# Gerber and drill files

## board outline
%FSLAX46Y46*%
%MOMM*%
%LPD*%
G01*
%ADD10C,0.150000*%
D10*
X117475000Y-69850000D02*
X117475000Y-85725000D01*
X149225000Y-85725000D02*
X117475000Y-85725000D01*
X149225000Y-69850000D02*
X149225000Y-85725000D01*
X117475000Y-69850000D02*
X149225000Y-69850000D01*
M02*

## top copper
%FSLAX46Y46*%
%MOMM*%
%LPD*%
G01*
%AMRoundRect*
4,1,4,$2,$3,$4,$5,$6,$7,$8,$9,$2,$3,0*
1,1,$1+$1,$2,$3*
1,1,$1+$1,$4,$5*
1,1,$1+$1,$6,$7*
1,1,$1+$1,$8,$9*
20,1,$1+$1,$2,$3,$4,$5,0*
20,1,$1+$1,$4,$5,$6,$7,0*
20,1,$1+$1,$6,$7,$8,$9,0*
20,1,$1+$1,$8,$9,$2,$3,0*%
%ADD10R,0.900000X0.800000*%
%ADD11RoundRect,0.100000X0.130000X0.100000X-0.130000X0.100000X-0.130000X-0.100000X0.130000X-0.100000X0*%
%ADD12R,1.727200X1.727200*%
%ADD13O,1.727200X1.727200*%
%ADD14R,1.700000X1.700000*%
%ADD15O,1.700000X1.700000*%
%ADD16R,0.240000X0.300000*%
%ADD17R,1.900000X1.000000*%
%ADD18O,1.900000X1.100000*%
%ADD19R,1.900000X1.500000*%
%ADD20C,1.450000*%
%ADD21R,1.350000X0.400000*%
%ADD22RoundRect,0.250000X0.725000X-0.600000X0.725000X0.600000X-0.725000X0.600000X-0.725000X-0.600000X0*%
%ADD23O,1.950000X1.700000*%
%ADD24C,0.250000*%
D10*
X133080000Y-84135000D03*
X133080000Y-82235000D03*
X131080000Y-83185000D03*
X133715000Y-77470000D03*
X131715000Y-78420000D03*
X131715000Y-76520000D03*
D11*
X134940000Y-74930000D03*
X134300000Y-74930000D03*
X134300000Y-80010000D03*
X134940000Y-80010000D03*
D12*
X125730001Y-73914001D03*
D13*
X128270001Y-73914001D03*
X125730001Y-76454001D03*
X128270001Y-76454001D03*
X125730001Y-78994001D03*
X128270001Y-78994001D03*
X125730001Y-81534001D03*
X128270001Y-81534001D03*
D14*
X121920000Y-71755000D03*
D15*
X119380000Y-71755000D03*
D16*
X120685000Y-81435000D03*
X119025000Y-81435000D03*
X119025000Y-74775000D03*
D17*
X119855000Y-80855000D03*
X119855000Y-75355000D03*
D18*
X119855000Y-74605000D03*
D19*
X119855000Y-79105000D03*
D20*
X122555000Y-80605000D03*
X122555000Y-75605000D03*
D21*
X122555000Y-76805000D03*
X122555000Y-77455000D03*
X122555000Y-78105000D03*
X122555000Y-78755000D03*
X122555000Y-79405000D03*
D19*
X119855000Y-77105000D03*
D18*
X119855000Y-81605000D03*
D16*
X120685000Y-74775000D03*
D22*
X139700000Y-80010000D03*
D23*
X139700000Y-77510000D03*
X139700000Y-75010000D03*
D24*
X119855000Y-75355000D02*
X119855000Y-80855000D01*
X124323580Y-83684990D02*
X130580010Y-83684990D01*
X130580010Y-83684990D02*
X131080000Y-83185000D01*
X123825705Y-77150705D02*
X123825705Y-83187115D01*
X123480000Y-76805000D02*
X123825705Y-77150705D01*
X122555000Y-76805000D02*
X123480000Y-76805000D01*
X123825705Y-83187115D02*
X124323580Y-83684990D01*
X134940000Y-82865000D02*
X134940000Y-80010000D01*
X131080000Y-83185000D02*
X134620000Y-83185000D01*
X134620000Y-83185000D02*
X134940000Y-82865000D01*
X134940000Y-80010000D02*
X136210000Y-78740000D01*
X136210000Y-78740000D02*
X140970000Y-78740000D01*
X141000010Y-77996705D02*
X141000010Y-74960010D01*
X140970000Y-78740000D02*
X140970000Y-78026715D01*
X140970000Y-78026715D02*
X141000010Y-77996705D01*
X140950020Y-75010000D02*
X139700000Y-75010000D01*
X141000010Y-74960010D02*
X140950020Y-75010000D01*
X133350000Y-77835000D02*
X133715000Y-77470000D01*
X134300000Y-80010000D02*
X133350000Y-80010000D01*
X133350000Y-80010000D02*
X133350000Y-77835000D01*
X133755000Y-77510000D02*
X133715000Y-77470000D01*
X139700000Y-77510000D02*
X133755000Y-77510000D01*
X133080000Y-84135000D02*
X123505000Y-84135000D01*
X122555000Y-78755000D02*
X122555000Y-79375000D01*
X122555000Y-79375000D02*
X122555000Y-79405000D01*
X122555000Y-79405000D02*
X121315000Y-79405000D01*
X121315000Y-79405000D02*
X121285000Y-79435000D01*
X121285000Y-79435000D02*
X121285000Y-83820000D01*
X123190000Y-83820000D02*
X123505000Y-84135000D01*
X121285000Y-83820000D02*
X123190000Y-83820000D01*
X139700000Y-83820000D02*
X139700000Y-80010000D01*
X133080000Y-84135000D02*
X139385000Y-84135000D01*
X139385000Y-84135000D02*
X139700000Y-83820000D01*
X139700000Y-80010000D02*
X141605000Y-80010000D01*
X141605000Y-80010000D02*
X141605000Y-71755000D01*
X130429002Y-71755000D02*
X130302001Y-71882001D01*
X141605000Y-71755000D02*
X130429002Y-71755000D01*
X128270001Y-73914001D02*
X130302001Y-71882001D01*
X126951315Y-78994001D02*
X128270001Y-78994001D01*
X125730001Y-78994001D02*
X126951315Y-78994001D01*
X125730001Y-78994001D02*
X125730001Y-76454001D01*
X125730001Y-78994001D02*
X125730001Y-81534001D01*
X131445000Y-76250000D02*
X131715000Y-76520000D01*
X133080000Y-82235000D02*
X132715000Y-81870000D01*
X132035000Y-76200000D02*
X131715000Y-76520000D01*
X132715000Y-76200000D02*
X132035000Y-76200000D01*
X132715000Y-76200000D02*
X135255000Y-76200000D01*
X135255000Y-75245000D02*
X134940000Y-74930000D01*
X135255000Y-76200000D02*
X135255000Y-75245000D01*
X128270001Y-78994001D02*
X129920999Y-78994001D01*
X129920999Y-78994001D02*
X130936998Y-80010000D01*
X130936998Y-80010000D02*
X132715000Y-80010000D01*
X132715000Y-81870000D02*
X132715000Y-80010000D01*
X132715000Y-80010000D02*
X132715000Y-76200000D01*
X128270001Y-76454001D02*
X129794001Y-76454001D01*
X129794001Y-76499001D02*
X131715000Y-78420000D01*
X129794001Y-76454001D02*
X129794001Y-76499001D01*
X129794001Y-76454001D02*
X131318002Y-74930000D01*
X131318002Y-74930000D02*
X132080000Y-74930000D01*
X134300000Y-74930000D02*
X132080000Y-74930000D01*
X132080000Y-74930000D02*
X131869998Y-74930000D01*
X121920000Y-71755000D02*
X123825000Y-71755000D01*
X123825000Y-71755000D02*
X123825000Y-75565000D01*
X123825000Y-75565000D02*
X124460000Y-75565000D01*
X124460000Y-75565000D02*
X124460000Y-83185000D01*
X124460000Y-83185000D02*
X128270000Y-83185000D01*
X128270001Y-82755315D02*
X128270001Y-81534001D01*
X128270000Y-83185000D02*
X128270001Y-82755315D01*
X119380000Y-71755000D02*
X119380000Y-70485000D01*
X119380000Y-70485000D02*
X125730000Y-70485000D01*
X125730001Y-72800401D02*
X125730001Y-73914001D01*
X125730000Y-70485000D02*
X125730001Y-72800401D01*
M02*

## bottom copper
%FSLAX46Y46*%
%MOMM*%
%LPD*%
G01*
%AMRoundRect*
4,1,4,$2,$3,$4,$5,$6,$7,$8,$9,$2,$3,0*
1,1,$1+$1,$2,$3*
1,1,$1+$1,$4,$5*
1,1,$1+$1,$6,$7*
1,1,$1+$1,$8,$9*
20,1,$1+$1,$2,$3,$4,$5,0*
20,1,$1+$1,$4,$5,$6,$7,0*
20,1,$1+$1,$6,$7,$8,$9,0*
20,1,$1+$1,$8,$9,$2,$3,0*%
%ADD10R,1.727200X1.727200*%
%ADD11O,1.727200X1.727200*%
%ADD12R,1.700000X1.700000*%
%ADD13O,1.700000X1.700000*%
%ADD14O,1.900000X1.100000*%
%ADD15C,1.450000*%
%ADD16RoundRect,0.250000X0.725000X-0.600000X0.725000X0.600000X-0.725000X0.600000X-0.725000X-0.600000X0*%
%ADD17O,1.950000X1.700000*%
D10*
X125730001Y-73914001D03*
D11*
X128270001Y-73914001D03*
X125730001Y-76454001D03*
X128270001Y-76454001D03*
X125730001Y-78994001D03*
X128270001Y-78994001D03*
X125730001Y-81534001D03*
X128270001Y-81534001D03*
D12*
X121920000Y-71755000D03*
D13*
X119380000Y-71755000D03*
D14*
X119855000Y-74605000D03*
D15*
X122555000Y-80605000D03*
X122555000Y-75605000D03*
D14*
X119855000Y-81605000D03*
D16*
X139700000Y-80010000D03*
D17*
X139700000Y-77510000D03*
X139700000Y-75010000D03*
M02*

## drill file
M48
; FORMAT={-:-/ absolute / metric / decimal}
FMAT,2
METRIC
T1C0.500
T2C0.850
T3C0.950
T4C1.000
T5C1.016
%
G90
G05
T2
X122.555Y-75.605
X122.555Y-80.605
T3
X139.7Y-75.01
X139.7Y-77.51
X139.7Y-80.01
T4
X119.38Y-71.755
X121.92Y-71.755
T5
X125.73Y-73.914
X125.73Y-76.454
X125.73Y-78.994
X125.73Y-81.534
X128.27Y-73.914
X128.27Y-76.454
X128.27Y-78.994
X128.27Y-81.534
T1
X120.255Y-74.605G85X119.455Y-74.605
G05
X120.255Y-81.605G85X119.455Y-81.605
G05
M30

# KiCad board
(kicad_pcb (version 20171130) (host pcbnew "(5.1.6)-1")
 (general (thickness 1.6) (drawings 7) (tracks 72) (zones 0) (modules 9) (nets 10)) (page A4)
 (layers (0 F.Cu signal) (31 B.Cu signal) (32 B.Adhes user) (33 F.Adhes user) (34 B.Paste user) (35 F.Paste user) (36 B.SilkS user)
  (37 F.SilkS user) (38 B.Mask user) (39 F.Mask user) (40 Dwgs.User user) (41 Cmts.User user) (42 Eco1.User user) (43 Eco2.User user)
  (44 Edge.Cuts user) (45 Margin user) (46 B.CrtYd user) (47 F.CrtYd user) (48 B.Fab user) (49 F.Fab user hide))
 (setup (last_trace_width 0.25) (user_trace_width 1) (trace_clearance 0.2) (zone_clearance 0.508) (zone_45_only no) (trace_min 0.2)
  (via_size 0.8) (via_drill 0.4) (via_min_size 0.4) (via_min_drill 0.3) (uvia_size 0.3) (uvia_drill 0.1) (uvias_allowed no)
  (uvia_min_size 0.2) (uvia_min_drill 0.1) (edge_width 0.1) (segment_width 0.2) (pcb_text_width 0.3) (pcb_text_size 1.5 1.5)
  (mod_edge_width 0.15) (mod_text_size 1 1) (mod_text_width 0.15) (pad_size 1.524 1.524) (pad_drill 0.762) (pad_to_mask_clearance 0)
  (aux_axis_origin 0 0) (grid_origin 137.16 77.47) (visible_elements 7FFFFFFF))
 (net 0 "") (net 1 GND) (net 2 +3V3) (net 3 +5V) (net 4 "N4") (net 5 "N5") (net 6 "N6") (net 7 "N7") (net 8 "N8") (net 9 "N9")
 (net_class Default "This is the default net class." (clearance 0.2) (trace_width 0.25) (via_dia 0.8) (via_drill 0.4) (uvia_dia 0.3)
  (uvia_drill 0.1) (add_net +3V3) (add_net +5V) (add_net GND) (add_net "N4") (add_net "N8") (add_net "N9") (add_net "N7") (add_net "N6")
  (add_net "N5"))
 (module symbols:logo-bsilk (layer F.Cu) (at 133.35 77.47)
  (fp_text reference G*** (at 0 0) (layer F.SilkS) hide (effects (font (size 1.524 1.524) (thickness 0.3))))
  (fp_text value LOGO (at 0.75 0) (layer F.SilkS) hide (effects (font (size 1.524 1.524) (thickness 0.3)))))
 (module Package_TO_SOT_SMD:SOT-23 (layer F.Cu) (at 132.08 83.185 180)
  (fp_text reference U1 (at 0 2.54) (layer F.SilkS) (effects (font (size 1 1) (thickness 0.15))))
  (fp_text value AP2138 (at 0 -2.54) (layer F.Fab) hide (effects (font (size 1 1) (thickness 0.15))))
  (pad 1 smd rect (at -1 -0.95 180) (size 0.9 0.8) (layers F.Cu F.Paste F.Mask) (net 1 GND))
  (pad 2 smd rect (at -1 0.95 180) (size 0.9 0.8) (layers F.Cu F.Paste F.Mask) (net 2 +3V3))
  (pad 3 smd rect (at 1 0 180) (size 0.9 0.8) (layers F.Cu F.Paste F.Mask) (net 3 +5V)))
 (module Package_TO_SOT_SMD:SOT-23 (layer F.Cu) (at 132.715 77.47)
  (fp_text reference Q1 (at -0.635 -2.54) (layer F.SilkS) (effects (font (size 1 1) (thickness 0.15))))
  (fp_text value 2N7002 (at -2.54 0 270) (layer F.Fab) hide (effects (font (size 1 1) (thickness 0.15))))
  (pad 3 smd rect (at 1 0) (size 0.9 0.8) (layers F.Cu F.Paste F.Mask) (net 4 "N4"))
  (pad 2 smd rect (at -1 0.95) (size 0.9 0.8) (layers F.Cu F.Paste F.Mask) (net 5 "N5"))
  (pad 1 smd rect (at -1 -0.95) (size 0.9 0.8) (layers F.Cu F.Paste F.Mask) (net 2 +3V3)))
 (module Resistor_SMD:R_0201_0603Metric (layer F.Cu) (at 134.62 74.93 180)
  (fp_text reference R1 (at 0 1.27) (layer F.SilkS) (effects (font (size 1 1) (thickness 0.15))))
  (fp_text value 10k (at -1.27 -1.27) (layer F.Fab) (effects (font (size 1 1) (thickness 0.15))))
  (pad "" smd roundrect (at -0.345 0 180) (size 0.318 0.36) (layers F.Paste) (roundrect_rratio 0.25))
  (pad "" smd roundrect (at 0.345 0 180) (size 0.318 0.36) (layers F.Paste) (roundrect_rratio 0.25))
  (pad 1 smd roundrect (at -0.32 0 180) (size 0.46 0.4) (layers F.Cu F.Mask) (roundrect_rratio 0.25) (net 2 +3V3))
  (pad 2 smd roundrect (at 0.32 0 180) (size 0.46 0.4) (layers F.Cu F.Mask) (roundrect_rratio 0.25) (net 5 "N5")))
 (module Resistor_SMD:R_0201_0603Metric (layer F.Cu) (at 134.62 80.01 180)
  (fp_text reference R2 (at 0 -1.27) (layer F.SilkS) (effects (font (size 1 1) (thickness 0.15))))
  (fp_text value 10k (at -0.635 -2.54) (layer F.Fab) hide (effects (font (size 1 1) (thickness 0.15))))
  (pad 2 smd roundrect (at 0.32 0 180) (size 0.46 0.4) (layers F.Cu F.Mask) (roundrect_rratio 0.25) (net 4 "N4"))
  (pad 1 smd roundrect (at -0.32 0 180) (size 0.46 0.4) (layers F.Cu F.Mask) (roundrect_rratio 0.25) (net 3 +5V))
  (pad "" smd roundrect (at 0.345 0 180) (size 0.318 0.36) (layers F.Paste) (roundrect_rratio 0.25))
  (pad "" smd roundrect (at -0.345 0 180) (size 0.318 0.36) (layers F.Paste) (roundrect_rratio 0.25)))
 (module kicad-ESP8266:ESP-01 (layer F.Cu) (at 125.730001 73.914001)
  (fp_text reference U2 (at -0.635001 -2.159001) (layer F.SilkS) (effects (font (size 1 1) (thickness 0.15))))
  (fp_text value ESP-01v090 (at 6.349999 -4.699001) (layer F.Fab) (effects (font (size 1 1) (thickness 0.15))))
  (pad 1 thru_hole rect (at 0 0) (size 1.7272 1.7272) (drill 1.016) (layers *.Cu *.Mask F.SilkS) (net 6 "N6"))
  (pad 2 thru_hole oval (at 2.54 0) (size 1.7272 1.7272) (drill 1.016) (layers *.Cu *.Mask F.SilkS) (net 1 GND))
  (pad 3 thru_hole oval (at 0 2.54) (size 1.7272 1.7272) (drill 1.016) (layers *.Cu *.Mask F.SilkS) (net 2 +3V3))
  (pad 4 thru_hole oval (at 2.54 2.54) (size 1.7272 1.7272) (drill 1.016) (layers *.Cu *.Mask F.SilkS) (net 5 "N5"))
  (pad 5 thru_hole oval (at 0 5.08) (size 1.7272 1.7272) (drill 1.016) (layers *.Cu *.Mask F.SilkS) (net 2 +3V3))
  (pad 6 thru_hole oval (at 2.54 5.08) (size 1.7272 1.7272) (drill 1.016) (layers *.Cu *.Mask F.SilkS) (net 2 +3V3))
  (pad 7 thru_hole oval (at 0 7.62) (size 1.7272 1.7272) (drill 1.016) (layers *.Cu *.Mask F.SilkS) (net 2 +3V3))
  (pad 8 thru_hole oval (at 2.54 7.62) (size 1.7272 1.7272) (drill 1.016) (layers *.Cu *.Mask F.SilkS) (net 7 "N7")))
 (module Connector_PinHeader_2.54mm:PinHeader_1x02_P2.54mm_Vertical (layer F.Cu) (at 121.92 71.755 270)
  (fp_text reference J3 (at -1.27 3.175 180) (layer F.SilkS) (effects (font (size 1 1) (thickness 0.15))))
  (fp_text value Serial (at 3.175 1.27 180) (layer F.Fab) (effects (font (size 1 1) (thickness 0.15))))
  (pad 1 thru_hole rect (at 0 0 270) (size 1.7 1.7) (drill 1) (layers *.Cu *.Mask) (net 7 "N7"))
  (pad 2 thru_hole oval (at 0 2.54 270) (size 1.7 1.7) (drill 1) (layers *.Cu *.Mask) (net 6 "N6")))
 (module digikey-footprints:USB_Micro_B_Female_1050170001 (layer F.Cu) (at 122.555 78.105 270)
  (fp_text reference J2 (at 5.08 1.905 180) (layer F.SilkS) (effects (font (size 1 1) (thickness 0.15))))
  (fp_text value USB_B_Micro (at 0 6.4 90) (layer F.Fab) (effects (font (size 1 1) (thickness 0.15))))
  (pad SH smd rect (at 3.33 1.87 270) (size 0.3 0.24) (layers F.Cu F.Paste F.Mask))
  (pad SH smd rect (at 3.33 3.53 270) (size 0.3 0.24) (layers F.Cu F.Paste F.Mask))
  (pad SH smd rect (at -3.33 3.53 270) (size 0.3 0.24) (layers F.Cu F.Paste F.Mask))
  (pad SH smd rect (at 2.75 2.7 270) (size 1 1.9) (layers F.Cu F.Paste F.Mask))
  (pad SH smd rect (at -2.75 2.7 270) (size 1 1.9) (layers F.Cu F.Paste F.Mask))
  (pad SH thru_hole oval (at -3.5 2.7 270) (size 1.1 1.9) (drill oval 0.5 1.3) (layers *.Cu *.Mask))
  (pad SH smd rect (at 1 2.7 270) (size 1.5 1.9) (layers F.Cu F.Paste F.Mask))
  (pad SH thru_hole circle (at 2.5 0 270) (size 1.45 1.45) (drill 0.85) (layers *.Cu *.Mask))
  (pad SH thru_hole circle (at -2.5 0 270) (size 1.45 1.45) (drill 0.85) (layers *.Cu *.Mask))
  (pad 1 smd rect (at -1.3 0 270) (size 0.4 1.35) (layers F.Cu F.Paste F.Mask) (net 3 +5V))
  (pad 2 smd rect (at -0.65 0 270) (size 0.4 1.35) (layers F.Cu F.Paste F.Mask) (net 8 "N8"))
  (pad 3 smd rect (at 0 0 270) (size 0.4 1.35) (layers F.Cu F.Paste F.Mask) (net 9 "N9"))
  (pad 4 smd rect (at 0.65 0 270) (size 0.4 1.35) (layers F.Cu F.Paste F.Mask) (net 1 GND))
  (pad 5 smd rect (at 1.3 0 270) (size 0.4 1.35) (layers F.Cu F.Paste F.Mask) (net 1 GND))
  (pad SH smd rect (at -1 2.7 270) (size 1.5 1.9) (layers F.Cu F.Paste F.Mask))
  (pad SH thru_hole oval (at 3.5 2.7 270) (size 1.1 1.9) (drill oval 0.5 1.3) (layers *.Cu *.Mask))
  (pad SH smd rect (at -3.33 1.87 270) (size 0.3 0.24) (layers F.Cu F.Paste F.Mask)))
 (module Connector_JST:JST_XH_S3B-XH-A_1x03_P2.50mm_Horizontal (layer F.Cu) (at 139.7 80.01 90)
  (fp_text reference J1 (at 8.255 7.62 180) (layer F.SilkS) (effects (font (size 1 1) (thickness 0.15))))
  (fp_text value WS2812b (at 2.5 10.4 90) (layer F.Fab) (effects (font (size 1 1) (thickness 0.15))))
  (pad 1 thru_hole roundrect (at 0 0 90) (size 1.7 1.95) (drill 0.95) (layers *.Cu *.Mask) (roundrect_rratio 0.147059) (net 1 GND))
  (pad 2 thru_hole oval (at 2.5 0 90) (size 1.7 1.95) (drill 0.95) (layers *.Cu *.Mask) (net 4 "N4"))
  (pad 3 thru_hole oval (at 5 0 90) (size 1.7 1.95) (drill 0.95) (layers *.Cu *.Mask) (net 3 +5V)))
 (gr_line (start 117.475 69.85) (end 117.475 85.725) (layer Edge.Cuts) (width 0.15))
 (gr_line (start 149.225 85.725) (end 117.475 85.725) (layer Edge.Cuts) (width 0.15))
 (gr_line (start 149.225 69.85) (end 149.225 85.725) (layer Edge.Cuts) (width 0.15))
 (gr_line (start 117.475 69.85) (end 149.225 69.85) (layer Edge.Cuts) (width 0.15))
 (segment (start 119.855 75.355) (end 119.855 80.855) (width 0.25) (layer F.Cu) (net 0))
 (segment (start 124.32358 83.68499) (end 130.58001 83.68499) (width 0.25) (layer F.Cu) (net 3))
 (segment (start 130.58001 83.68499) (end 131.08 83.185) (width 0.25) (layer F.Cu) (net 3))
 (segment (start 123.825705 77.150705) (end 123.825705 83.187115) (width 0.25) (layer F.Cu) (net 3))
 (segment (start 123.48 76.805) (end 123.825705 77.150705) (width 0.25) (layer F.Cu) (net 3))
 (segment (start 122.555 76.805) (end 123.48 76.805) (width 0.25) (layer F.Cu) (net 3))
 (segment (start 123.825705 83.187115) (end 124.32358 83.68499) (width 0.25) (layer F.Cu) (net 3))
 (segment (start 134.94 82.865) (end 134.94 80.01) (width 0.25) (layer F.Cu) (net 3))
 (segment (start 131.08 83.185) (end 134.62 83.185) (width 0.25) (layer F.Cu) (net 3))
 (segment (start 134.62 83.185) (end 134.94 82.865) (width 0.25) (layer F.Cu) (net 3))
 (segment (start 134.94 80.01) (end 136.21 78.74) (width 0.25) (layer F.Cu) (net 3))
 (segment (start 136.21 78.74) (end 140.97 78.74) (width 0.25) (layer F.Cu) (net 3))
 (segment (start 141.00001 77.996705) (end 141.00001 74.96001) (width 0.25) (layer F.Cu) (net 3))
 (segment (start 140.97 78.74) (end 140.97 78.026715) (width 0.25) (layer F.Cu) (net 3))
 (segment (start 140.97 78.026715) (end 141.00001 77.996705) (width 0.25) (layer F.Cu) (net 3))
 (segment (start 140.95002 75.01) (end 139.7 75.01) (width 0.25) (layer F.Cu) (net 3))
 (segment (start 141.00001 74.96001) (end 140.95002 75.01) (width 0.25) (layer F.Cu) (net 3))
 (segment (start 133.35 77.835) (end 133.715 77.47) (width 0.25) (layer F.Cu) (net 4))
 (segment (start 134.3 80.01) (end 133.35 80.01) (width 0.25) (layer F.Cu) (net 4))
 (segment (start 133.35 80.01) (end 133.35 77.835) (width 0.25) (layer F.Cu) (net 4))
 (segment (start 133.755 77.51) (end 133.715 77.47) (width 0.25) (layer F.Cu) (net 4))
 (segment (start 139.7 77.51) (end 133.755 77.51) (width 0.25) (layer F.Cu) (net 4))
 (segment (start 133.08 84.135) (end 123.505 84.135) (width 0.25) (layer F.Cu) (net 1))
 (segment (start 122.555 78.755) (end 122.555 79.375) (width 0.25) (layer F.Cu) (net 1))
 (segment (start 122.555 79.375) (end 122.555 79.405) (width 0.25) (layer F.Cu) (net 1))
 (segment (start 122.555 79.405) (end 121.315 79.405) (width 0.25) (layer F.Cu) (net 1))
 (segment (start 121.315 79.405) (end 121.285 79.435) (width 0.25) (layer F.Cu) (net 1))
 (segment (start 121.285 79.435) (end 121.285 83.82) (width 0.25) (layer F.Cu) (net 1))
 (segment (start 123.19 83.82) (end 123.505 84.135) (width 0.25) (layer F.Cu) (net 1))
 (segment (start 121.285 83.82) (end 123.19 83.82) (width 0.25) (layer F.Cu) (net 1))
 (segment (start 139.7 83.82) (end 139.7 80.01) (width 0.25) (layer F.Cu) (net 1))
 (segment (start 133.08 84.135) (end 139.385 84.135) (width 0.25) (layer F.Cu) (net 1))
 (segment (start 139.385 84.135) (end 139.7 83.82) (width 0.25) (layer F.Cu) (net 1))
 (segment (start 139.7 80.01) (end 141.605 80.01) (width 0.25) (layer F.Cu) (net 1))
 (segment (start 141.605 80.01) (end 141.605 71.755) (width 0.25) (layer F.Cu) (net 1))
 (segment (start 130.429002 71.755) (end 130.302001 71.882001) (width 0.25) (layer F.Cu) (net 1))
 (segment (start 141.605 71.755) (end 130.429002 71.755) (width 0.25) (layer F.Cu) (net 1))
 (segment (start 128.270001 73.914001) (end 130.302001 71.882001) (width 0.25) (layer F.Cu) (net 1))
 (segment (start 126.951315 78.994001) (end 128.270001 78.994001) (width 0.25) (layer F.Cu) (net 2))
 (segment (start 125.730001 78.994001) (end 126.951315 78.994001) (width 0.25) (layer F.Cu) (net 2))
 (segment (start 125.730001 78.994001) (end 125.730001 76.454001) (width 0.25) (layer F.Cu) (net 2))
 (segment (start 125.730001 78.994001) (end 125.730001 81.534001) (width 0.25) (layer F.Cu) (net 2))
 (segment (start 131.445 76.25) (end 131.715 76.52) (width 0.25) (layer F.Cu) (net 2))
 (segment (start 133.08 82.235) (end 132.715 81.87) (width 0.25) (layer F.Cu) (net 2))
 (segment (start 132.035 76.2) (end 131.715 76.52) (width 0.25) (layer F.Cu) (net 2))
 (segment (start 132.715 76.2) (end 132.035 76.2) (width 0.25) (layer F.Cu) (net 2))
 (segment (start 132.715 76.2) (end 135.255 76.2) (width 0.25) (layer F.Cu) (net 2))
 (segment (start 135.255 75.245) (end 134.94 74.93) (width 0.25) (layer F.Cu) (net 2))
 (segment (start 135.255 76.2) (end 135.255 75.245) (width 0.25) (layer F.Cu) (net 2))
 (segment (start 128.270001 78.994001) (end 129.920999 78.994001) (width 0.25) (layer F.Cu) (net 2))
 (segment (start 129.920999 78.994001) (end 130.936998 80.01) (width 0.25) (layer F.Cu) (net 2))
 (segment (start 130.936998 80.01) (end 132.715 80.01) (width 0.25) (layer F.Cu) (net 2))
 (segment (start 132.715 81.87) (end 132.715 80.01) (width 0.25) (layer F.Cu) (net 2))
 (segment (start 132.715 80.01) (end 132.715 76.2) (width 0.25) (layer F.Cu) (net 2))
 (segment (start 128.270001 76.454001) (end 129.794001 76.454001) (width 0.25) (layer F.Cu) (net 5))
 (segment (start 129.794001 76.499001) (end 131.715 78.42) (width 0.25) (layer F.Cu) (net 5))
 (segment (start 129.794001 76.454001) (end 129.794001 76.499001) (width 0.25) (layer F.Cu) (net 5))
 (segment (start 129.794001 76.454001) (end 131.318002 74.93) (width 0.25) (layer F.Cu) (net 5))
 (segment (start 131.318002 74.93) (end 132.08 74.93) (width 0.25) (layer F.Cu) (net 5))
 (segment (start 134.3 74.93) (end 132.08 74.93) (width 0.25) (layer F.Cu) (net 5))
 (segment (start 132.08 74.93) (end 131.869998 74.93) (width 0.25) (layer F.Cu) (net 5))
 (segment (start 121.92 71.755) (end 123.825 71.755) (width 0.25) (layer F.Cu) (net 7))
 (segment (start 123.825 71.755) (end 123.825 75.565) (width 0.25) (layer F.Cu) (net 7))
 (segment (start 123.825 75.565) (end 124.46 75.565) (width 0.25) (layer F.Cu) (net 7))
 (segment (start 124.46 75.565) (end 124.46 83.185) (width 0.25) (layer F.Cu) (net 7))
 (segment (start 124.46 83.185) (end 128.27 83.185) (width 0.25) (layer F.Cu) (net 7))
 (segment (start 128.270001 82.755315) (end 128.270001 81.534001) (width 0.25) (layer F.Cu) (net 7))
 (segment (start 128.27 83.185) (end 128.270001 82.755315) (width 0.25) (layer F.Cu) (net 7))
 (segment (start 119.38 71.755) (end 119.38 70.485) (width 0.25) (layer F.Cu) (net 6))
 (segment (start 119.38 70.485) (end 125.73 70.485) (width 0.25) (layer F.Cu) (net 6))
 (segment (start 125.730001 72.800401) (end 125.730001 73.914001) (width 0.25) (layer F.Cu) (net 6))
 (segment (start 125.73 70.485) (end 125.730001 72.800401) (width 0.25) (layer F.Cu) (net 6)))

